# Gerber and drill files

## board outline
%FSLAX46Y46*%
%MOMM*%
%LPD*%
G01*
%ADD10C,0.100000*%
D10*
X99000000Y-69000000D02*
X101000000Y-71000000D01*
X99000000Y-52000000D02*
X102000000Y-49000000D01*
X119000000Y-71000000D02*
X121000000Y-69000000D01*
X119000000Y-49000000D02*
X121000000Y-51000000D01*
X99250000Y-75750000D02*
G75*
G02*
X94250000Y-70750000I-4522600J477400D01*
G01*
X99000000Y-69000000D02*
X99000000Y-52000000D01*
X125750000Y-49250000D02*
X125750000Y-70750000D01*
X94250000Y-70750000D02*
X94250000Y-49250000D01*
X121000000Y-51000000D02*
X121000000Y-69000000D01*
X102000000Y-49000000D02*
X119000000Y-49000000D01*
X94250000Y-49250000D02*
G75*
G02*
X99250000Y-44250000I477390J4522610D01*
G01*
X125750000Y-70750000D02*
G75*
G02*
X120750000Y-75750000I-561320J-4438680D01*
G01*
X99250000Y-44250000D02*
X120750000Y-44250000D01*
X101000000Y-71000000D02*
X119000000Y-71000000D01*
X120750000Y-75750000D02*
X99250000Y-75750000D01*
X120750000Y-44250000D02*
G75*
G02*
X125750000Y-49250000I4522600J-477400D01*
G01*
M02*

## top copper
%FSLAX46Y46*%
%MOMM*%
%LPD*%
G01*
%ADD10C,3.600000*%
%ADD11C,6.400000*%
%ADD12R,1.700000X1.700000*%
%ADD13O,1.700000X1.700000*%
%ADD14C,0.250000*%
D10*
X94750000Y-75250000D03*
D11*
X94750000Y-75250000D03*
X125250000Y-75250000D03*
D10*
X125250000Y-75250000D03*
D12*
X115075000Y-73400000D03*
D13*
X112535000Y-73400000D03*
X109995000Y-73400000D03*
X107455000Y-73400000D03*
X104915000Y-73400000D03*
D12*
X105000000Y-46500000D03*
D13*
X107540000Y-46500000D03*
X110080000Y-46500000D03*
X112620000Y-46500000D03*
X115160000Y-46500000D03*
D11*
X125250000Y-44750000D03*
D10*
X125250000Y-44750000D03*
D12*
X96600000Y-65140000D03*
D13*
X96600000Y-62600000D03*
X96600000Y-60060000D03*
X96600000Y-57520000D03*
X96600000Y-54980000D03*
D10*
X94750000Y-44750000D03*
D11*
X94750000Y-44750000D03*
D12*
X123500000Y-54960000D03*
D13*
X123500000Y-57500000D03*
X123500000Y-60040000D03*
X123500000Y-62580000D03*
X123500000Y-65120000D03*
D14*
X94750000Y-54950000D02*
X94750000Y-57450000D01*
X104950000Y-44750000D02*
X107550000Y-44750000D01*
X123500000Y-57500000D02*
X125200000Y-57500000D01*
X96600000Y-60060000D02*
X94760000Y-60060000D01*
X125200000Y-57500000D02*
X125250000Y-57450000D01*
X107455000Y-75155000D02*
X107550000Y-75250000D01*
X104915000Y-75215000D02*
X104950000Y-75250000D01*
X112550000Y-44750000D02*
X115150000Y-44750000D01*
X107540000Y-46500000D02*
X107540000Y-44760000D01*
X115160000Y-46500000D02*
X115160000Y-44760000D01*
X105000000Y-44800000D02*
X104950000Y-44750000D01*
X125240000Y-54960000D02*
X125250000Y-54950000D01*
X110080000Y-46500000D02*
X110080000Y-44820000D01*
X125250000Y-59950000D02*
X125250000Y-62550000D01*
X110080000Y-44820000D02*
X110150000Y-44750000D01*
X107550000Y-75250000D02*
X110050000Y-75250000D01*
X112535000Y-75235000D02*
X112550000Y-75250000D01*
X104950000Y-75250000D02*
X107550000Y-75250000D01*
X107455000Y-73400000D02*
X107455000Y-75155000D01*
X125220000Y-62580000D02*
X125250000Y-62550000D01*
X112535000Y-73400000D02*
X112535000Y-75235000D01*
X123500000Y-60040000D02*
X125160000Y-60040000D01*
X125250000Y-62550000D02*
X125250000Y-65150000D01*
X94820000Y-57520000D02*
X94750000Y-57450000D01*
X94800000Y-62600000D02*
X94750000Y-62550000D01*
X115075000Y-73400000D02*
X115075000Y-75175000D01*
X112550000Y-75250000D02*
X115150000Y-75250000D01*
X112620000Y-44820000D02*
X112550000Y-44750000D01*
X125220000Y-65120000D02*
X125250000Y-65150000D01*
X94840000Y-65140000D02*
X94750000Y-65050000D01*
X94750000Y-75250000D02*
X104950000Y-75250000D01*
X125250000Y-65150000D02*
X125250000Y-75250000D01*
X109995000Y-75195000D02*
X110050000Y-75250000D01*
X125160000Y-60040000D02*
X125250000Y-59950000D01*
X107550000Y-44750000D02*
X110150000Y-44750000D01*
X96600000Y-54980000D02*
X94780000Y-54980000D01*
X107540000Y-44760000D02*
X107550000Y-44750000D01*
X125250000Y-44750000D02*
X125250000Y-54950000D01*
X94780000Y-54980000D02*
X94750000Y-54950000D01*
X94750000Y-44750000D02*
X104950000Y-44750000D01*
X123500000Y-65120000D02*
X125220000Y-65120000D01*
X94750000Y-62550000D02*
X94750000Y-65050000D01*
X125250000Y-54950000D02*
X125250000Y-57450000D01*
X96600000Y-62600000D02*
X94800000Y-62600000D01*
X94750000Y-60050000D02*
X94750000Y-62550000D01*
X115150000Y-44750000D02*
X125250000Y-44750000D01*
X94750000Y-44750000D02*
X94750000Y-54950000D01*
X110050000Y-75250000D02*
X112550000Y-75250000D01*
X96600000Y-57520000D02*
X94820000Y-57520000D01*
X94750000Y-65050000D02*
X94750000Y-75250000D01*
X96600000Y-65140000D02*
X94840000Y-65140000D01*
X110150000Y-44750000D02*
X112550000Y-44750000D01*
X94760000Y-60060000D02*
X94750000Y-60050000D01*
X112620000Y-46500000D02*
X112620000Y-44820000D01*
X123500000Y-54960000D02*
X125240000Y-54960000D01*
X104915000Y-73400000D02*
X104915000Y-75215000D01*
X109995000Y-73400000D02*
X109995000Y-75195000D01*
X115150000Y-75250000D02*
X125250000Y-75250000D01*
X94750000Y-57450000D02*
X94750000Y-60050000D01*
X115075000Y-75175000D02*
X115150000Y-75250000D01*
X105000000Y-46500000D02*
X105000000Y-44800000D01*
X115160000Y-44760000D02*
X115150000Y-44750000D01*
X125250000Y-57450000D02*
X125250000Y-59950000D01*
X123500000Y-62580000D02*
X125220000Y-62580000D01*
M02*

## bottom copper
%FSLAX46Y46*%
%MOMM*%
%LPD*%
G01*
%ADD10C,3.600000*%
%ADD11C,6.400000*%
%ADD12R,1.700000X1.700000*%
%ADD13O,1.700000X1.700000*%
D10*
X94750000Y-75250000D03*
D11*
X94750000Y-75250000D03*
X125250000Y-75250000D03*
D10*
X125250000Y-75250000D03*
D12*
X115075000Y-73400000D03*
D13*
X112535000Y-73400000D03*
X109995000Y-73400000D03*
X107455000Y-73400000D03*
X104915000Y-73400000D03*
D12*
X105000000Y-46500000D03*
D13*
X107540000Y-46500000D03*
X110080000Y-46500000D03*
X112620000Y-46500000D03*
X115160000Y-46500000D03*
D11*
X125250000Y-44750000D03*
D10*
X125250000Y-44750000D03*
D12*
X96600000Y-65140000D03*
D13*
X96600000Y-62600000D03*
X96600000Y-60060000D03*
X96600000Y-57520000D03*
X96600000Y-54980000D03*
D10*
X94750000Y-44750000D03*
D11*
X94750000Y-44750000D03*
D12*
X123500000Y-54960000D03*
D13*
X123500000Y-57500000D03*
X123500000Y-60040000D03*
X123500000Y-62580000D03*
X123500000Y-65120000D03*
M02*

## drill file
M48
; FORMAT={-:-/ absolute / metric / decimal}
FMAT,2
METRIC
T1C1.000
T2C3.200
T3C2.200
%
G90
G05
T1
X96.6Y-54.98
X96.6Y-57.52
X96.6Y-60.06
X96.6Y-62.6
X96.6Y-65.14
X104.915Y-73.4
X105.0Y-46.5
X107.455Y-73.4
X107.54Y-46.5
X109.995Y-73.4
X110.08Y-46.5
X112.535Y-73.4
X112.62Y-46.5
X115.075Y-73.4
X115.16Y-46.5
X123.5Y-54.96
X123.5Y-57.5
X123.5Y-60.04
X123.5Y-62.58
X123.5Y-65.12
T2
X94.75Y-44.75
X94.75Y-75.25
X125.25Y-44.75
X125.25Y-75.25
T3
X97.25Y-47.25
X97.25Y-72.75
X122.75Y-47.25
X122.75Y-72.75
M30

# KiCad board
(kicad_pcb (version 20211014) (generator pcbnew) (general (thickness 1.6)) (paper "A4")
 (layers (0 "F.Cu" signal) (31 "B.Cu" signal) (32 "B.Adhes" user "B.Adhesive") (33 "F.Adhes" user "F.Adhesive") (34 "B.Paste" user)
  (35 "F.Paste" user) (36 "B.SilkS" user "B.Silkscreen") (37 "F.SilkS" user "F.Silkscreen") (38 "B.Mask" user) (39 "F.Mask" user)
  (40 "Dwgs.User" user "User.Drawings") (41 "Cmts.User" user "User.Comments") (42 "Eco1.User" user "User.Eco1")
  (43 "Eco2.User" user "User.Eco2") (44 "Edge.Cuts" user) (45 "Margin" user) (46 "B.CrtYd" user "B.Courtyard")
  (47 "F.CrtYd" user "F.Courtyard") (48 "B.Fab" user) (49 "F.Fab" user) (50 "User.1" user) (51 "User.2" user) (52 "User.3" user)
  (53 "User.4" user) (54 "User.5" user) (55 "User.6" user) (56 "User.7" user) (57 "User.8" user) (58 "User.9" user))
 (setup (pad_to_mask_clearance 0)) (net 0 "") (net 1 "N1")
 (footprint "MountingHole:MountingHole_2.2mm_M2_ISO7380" (layer "F.Cu") (at 122.75 47.25)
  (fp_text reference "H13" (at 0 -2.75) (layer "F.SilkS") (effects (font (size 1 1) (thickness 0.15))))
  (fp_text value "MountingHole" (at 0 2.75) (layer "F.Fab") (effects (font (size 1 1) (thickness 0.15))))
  (pad "" np_thru_hole circle (at 0 0) (size 2.2 2.2) (drill 2.2) (layers *.Cu *.Mask)))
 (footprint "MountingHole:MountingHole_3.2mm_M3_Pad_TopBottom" (layer "F.Cu") (at 94.75 75.25)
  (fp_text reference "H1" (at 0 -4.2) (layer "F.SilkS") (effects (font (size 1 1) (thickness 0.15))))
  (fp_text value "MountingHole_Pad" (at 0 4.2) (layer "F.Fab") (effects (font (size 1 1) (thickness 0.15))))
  (pad "1" thru_hole circle (at 0 0) (size 3.6 3.6) (drill 3.2) (layers *.Cu *.Mask) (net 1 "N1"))
  (pad "1" connect circle (at 0 0) (size 6.4 6.4) (layers "B.Cu" "B.Mask") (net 1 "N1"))
  (pad "1" connect circle (at 0 0) (size 6.4 6.4) (layers "F.Cu" "F.Mask") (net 1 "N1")))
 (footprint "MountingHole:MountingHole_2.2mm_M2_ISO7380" (layer "F.Cu") (at 97.25 72.75)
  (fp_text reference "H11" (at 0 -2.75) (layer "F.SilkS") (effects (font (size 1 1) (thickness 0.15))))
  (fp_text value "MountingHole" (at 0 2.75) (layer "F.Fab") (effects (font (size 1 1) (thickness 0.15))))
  (pad "" np_thru_hole circle (at 0 0) (size 2.2 2.2) (drill 2.2) (layers *.Cu *.Mask)))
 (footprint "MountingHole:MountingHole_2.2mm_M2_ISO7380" (layer "F.Cu") (at 97.25 47.25)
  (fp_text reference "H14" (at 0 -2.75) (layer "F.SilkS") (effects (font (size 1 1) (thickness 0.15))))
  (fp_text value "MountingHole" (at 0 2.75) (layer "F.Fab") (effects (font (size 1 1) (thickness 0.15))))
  (pad "" np_thru_hole circle (at 0 0) (size 2.2 2.2) (drill 2.2) (layers *.Cu *.Mask)))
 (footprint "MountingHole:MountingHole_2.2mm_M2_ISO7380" (layer "F.Cu") (at 122.75 72.75)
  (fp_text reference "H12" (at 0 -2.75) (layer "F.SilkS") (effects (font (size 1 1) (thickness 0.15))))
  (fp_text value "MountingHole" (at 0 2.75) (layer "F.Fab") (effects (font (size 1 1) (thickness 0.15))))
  (pad "" np_thru_hole circle (at 0 0) (size 2.2 2.2) (drill 2.2) (layers *.Cu *.Mask)))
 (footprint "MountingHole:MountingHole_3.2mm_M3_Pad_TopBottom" (layer "F.Cu") (at 125.25 75.25)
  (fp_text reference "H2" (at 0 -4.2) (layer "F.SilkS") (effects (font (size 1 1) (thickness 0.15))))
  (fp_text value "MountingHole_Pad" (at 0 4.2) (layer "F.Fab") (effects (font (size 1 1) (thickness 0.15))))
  (pad "1" connect circle (at 0 0) (size 6.4 6.4) (layers "B.Cu" "B.Mask") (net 1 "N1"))
  (pad "1" connect circle (at 0 0) (size 6.4 6.4) (layers "F.Cu" "F.Mask") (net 1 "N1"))
  (pad "1" thru_hole circle (at 0 0) (size 3.6 3.6) (drill 3.2) (layers *.Cu *.Mask) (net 1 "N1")))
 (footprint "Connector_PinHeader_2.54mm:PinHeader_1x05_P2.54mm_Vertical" (layer "F.Cu") (at 115.075 73.4 -90)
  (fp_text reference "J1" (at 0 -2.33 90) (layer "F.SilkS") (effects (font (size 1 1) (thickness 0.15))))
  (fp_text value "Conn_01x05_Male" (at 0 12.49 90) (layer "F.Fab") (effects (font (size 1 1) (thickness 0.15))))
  (pad "1" thru_hole rect (at 0 0 270) (size 1.7 1.7) (drill 1) (layers *.Cu *.Mask) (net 1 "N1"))
  (pad "2" thru_hole oval (at 0 2.54 270) (size 1.7 1.7) (drill 1) (layers *.Cu *.Mask) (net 1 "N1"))
  (pad "3" thru_hole oval (at 0 5.08 270) (size 1.7 1.7) (drill 1) (layers *.Cu *.Mask) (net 1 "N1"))
  (pad "4" thru_hole oval (at 0 7.62 270) (size 1.7 1.7) (drill 1) (layers *.Cu *.Mask) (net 1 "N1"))
  (pad "5" thru_hole oval (at 0 10.16 270) (size 1.7 1.7) (drill 1) (layers *.Cu *.Mask) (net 1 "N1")))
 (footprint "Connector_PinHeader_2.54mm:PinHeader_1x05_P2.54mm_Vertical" (layer "F.Cu") (at 105 46.5 90)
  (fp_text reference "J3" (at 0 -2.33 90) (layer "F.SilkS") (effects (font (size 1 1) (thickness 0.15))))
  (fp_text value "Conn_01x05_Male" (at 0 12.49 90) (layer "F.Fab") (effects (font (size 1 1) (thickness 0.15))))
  (pad "1" thru_hole rect (at 0 0 90) (size 1.7 1.7) (drill 1) (layers *.Cu *.Mask) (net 1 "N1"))
  (pad "2" thru_hole oval (at 0 2.54 90) (size 1.7 1.7) (drill 1) (layers *.Cu *.Mask) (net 1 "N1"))
  (pad "3" thru_hole oval (at 0 5.08 90) (size 1.7 1.7) (drill 1) (layers *.Cu *.Mask) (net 1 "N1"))
  (pad "4" thru_hole oval (at 0 7.62 90) (size 1.7 1.7) (drill 1) (layers *.Cu *.Mask) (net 1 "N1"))
  (pad "5" thru_hole oval (at 0 10.16 90) (size 1.7 1.7) (drill 1) (layers *.Cu *.Mask) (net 1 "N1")))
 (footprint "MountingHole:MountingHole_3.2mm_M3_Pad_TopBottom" (layer "F.Cu") (at 125.25 44.75)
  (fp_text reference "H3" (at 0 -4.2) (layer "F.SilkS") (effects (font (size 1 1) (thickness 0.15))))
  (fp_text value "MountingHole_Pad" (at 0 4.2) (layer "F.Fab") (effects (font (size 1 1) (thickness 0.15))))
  (pad "1" connect circle (at 0 0) (size 6.4 6.4) (layers "F.Cu" "F.Mask") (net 1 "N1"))
  (pad "1" connect circle (at 0 0) (size 6.4 6.4) (layers "B.Cu" "B.Mask") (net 1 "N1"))
  (pad "1" thru_hole circle (at 0 0) (size 3.6 3.6) (drill 3.2) (layers *.Cu *.Mask) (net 1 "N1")))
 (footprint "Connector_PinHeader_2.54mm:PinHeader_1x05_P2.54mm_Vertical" (layer "F.Cu") (at 96.6 65.14 180)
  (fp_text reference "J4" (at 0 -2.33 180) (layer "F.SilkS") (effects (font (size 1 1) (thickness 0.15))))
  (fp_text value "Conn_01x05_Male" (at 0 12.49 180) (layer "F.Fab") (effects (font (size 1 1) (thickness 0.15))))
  (pad "1" thru_hole rect (at 0 0 180) (size 1.7 1.7) (drill 1) (layers *.Cu *.Mask) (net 1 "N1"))
  (pad "2" thru_hole oval (at 0 2.54 180) (size 1.7 1.7) (drill 1) (layers *.Cu *.Mask) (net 1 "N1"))
  (pad "3" thru_hole oval (at 0 5.08 180) (size 1.7 1.7) (drill 1) (layers *.Cu *.Mask) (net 1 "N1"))
  (pad "4" thru_hole oval (at 0 7.62 180) (size 1.7 1.7) (drill 1) (layers *.Cu *.Mask) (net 1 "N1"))
  (pad "5" thru_hole oval (at 0 10.16 180) (size 1.7 1.7) (drill 1) (layers *.Cu *.Mask) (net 1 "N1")))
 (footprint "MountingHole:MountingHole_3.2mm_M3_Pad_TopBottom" (layer "F.Cu") (at 94.75 44.75)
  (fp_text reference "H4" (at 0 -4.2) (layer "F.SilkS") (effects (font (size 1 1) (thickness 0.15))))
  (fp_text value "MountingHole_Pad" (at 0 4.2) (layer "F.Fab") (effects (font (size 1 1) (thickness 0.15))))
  (pad "1" thru_hole circle (at 0 0) (size 3.6 3.6) (drill 3.2) (layers *.Cu *.Mask) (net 1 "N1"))
  (pad "1" connect circle (at 0 0) (size 6.4 6.4) (layers "F.Cu" "F.Mask") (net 1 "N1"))
  (pad "1" connect circle (at 0 0) (size 6.4 6.4) (layers "B.Cu" "B.Mask") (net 1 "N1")))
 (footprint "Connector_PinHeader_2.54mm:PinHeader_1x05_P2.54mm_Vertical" (layer "F.Cu") (at 123.5 54.96)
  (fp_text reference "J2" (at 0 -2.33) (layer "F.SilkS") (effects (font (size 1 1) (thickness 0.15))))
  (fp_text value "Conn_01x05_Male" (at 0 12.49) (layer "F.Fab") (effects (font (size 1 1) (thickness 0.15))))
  (pad "1" thru_hole rect (at 0 0) (size 1.7 1.7) (drill 1) (layers *.Cu *.Mask) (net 1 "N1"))
  (pad "2" thru_hole oval (at 0 2.54) (size 1.7 1.7) (drill 1) (layers *.Cu *.Mask) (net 1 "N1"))
  (pad "3" thru_hole oval (at 0 5.08) (size 1.7 1.7) (drill 1) (layers *.Cu *.Mask) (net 1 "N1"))
  (pad "4" thru_hole oval (at 0 7.62) (size 1.7 1.7) (drill 1) (layers *.Cu *.Mask) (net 1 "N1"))
  (pad "5" thru_hole oval (at 0 10.16) (size 1.7 1.7) (drill 1) (layers *.Cu *.Mask) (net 1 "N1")))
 (gr_line (start 99 69) (end 101 71) (layer "Edge.Cuts") (width 0.1))
 (gr_line (start 99 52) (end 102 49) (layer "Edge.Cuts") (width 0.1))
 (gr_line (start 119 71) (end 121 69) (layer "Edge.Cuts") (width 0.1))
 (gr_line (start 119 49) (end 121 51) (layer "Edge.Cuts") (width 0.1))
 (gr_arc (start 99.25 75.75) (mid 91.511648 78.48835) (end 94.25 70.75) (layer "Edge.Cuts") (width 0.1))
 (gr_line (start 99 69) (end 99 52) (layer "Edge.Cuts") (width 0.1))
 (gr_line (start 125.75 49.25) (end 125.75 70.75) (layer "Edge.Cuts") (width 0.1))
 (gr_line (start 94.25 70.75) (end 94.25 49.25) (layer "Edge.Cuts") (width 0.1))
 (gr_line (start 121 51) (end 121 69) (layer "Edge.Cuts") (width 0.1))
 (gr_line (start 102 49) (end 119 49) (layer "Edge.Cuts") (width 0.1))
 (gr_arc (start 94.25 49.25) (mid 91.511649 41.511649) (end 99.25 44.25) (layer "Edge.Cuts") (width 0.1))
 (gr_arc (start 125.75 70.75) (mid 128.352298 78.352298) (end 120.75 75.75) (layer "Edge.Cuts") (width 0.1))
 (gr_line (start 99.25 44.25) (end 120.75 44.25) (layer "Edge.Cuts") (width 0.1))
 (gr_line (start 101 71) (end 119 71) (layer "Edge.Cuts") (width 0.1))
 (gr_line (start 120.75 75.75) (end 99.25 75.75) (layer "Edge.Cuts") (width 0.1))
 (gr_arc (start 120.75 44.25) (mid 128.488349 41.511649) (end 125.75 49.25) (layer "Edge.Cuts") (width 0.1))
 (segment (start 94.75 54.95) (end 94.75 57.45) (width 0.25) (layer "F.Cu") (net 1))
 (segment (start 104.95 44.75) (end 107.55 44.75) (width 0.25) (layer "F.Cu") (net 1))
 (segment (start 123.5 57.5) (end 125.2 57.5) (width 0.25) (layer "F.Cu") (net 1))
 (segment (start 96.6 60.06) (end 94.76 60.06) (width 0.25) (layer "F.Cu") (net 1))
 (segment (start 125.2 57.5) (end 125.25 57.45) (width 0.25) (layer "F.Cu") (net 1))
 (segment (start 107.455 75.155) (end 107.55 75.25) (width 0.25) (layer "F.Cu") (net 1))
 (segment (start 104.915 75.215) (end 104.95 75.25) (width 0.25) (layer "F.Cu") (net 1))
 (segment (start 112.55 44.75) (end 115.15 44.75) (width 0.25) (layer "F.Cu") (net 1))
 (segment (start 107.54 46.5) (end 107.54 44.76) (width 0.25) (layer "F.Cu") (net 1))
 (segment (start 115.16 46.5) (end 115.16 44.76) (width 0.25) (layer "F.Cu") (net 1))
 (segment (start 105 44.8) (end 104.95 44.75) (width 0.25) (layer "F.Cu") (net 1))
 (segment (start 125.24 54.96) (end 125.25 54.95) (width 0.25) (layer "F.Cu") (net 1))
 (segment (start 110.08 46.5) (end 110.08 44.82) (width 0.25) (layer "F.Cu") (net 1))
 (segment (start 125.25 59.95) (end 125.25 62.55) (width 0.25) (layer "F.Cu") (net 1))
 (segment (start 110.08 44.82) (end 110.15 44.75) (width 0.25) (layer "F.Cu") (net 1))
 (segment (start 107.55 75.25) (end 110.05 75.25) (width 0.25) (layer "F.Cu") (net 1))
 (segment (start 112.535 75.235) (end 112.55 75.25) (width 0.25) (layer "F.Cu") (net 1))
 (segment (start 104.95 75.25) (end 107.55 75.25) (width 0.25) (layer "F.Cu") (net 1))
 (segment (start 107.455 73.4) (end 107.455 75.155) (width 0.25) (layer "F.Cu") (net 1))
 (segment (start 125.22 62.58) (end 125.25 62.55) (width 0.25) (layer "F.Cu") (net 1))
 (segment (start 112.535 73.4) (end 112.535 75.235) (width 0.25) (layer "F.Cu") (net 1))
 (segment (start 123.5 60.04) (end 125.16 60.04) (width 0.25) (layer "F.Cu") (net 1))
 (segment (start 125.25 62.55) (end 125.25 65.15) (width 0.25) (layer "F.Cu") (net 1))
 (segment (start 94.82 57.52) (end 94.75 57.45) (width 0.25) (layer "F.Cu") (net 1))
 (segment (start 94.8 62.6) (end 94.75 62.55) (width 0.25) (layer "F.Cu") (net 1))
 (segment (start 115.075 73.4) (end 115.075 75.175) (width 0.25) (layer "F.Cu") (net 1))
 (segment (start 112.55 75.25) (end 115.15 75.25) (width 0.25) (layer "F.Cu") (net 1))
 (segment (start 112.62 44.82) (end 112.55 44.75) (width 0.25) (layer "F.Cu") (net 1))
 (segment (start 125.22 65.12) (end 125.25 65.15) (width 0.25) (layer "F.Cu") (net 1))
 (segment (start 94.84 65.14) (end 94.75 65.05) (width 0.25) (layer "F.Cu") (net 1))
 (segment (start 94.75 75.25) (end 104.95 75.25) (width 0.25) (layer "F.Cu") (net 1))
 (segment (start 125.25 65.15) (end 125.25 75.25) (width 0.25) (layer "F.Cu") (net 1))
 (segment (start 109.995 75.195) (end 110.05 75.25) (width 0.25) (layer "F.Cu") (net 1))
 (segment (start 125.16 60.04) (end 125.25 59.95) (width 0.25) (layer "F.Cu") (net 1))
 (segment (start 107.55 44.75) (end 110.15 44.75) (width 0.25) (layer "F.Cu") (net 1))
 (segment (start 96.6 54.98) (end 94.78 54.98) (width 0.25) (layer "F.Cu") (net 1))
 (segment (start 107.54 44.76) (end 107.55 44.75) (width 0.25) (layer "F.Cu") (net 1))
 (segment (start 125.25 44.75) (end 125.25 54.95) (width 0.25) (layer "F.Cu") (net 1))
 (segment (start 94.78 54.98) (end 94.75 54.95) (width 0.25) (layer "F.Cu") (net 1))
 (segment (start 94.75 44.75) (end 104.95 44.75) (width 0.25) (layer "F.Cu") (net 1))
 (segment (start 123.5 65.12) (end 125.22 65.12) (width 0.25) (layer "F.Cu") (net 1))
 (segment (start 94.75 62.55) (end 94.75 65.05) (width 0.25) (layer "F.Cu") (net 1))
 (segment (start 125.25 54.95) (end 125.25 57.45) (width 0.25) (layer "F.Cu") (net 1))
 (segment (start 96.6 62.6) (end 94.8 62.6) (width 0.25) (layer "F.Cu") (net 1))
 (segment (start 94.75 60.05) (end 94.75 62.55) (width 0.25) (layer "F.Cu") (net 1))
 (segment (start 115.15 44.75) (end 125.25 44.75) (width 0.25) (layer "F.Cu") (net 1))
 (segment (start 94.75 44.75) (end 94.75 54.95) (width 0.25) (layer "F.Cu") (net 1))
 (segment (start 110.05 75.25) (end 112.55 75.25) (width 0.25) (layer "F.Cu") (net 1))
 (segment (start 96.6 57.52) (end 94.82 57.52) (width 0.25) (layer "F.Cu") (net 1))
 (segment (start 94.75 65.05) (end 94.75 75.25) (width 0.25) (layer "F.Cu") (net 1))
 (segment (start 96.6 65.14) (end 94.84 65.14) (width 0.25) (layer "F.Cu") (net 1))
 (segment (start 110.15 44.75) (end 112.55 44.75) (width 0.25) (layer "F.Cu") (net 1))
 (segment (start 94.76 60.06) (end 94.75 60.05) (width 0.25) (layer "F.Cu") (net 1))
 (segment (start 112.62 46.5) (end 112.62 44.82) (width 0.25) (layer "F.Cu") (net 1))
 (segment (start 123.5 54.96) (end 125.24 54.96) (width 0.25) (layer "F.Cu") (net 1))
 (segment (start 104.915 73.4) (end 104.915 75.215) (width 0.25) (layer "F.Cu") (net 1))
 (segment (start 109.995 73.4) (end 109.995 75.195) (width 0.25) (layer "F.Cu") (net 1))
 (segment (start 115.15 75.25) (end 125.25 75.25) (width 0.25) (layer "F.Cu") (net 1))
 (segment (start 94.75 57.45) (end 94.75 60.05) (width 0.25) (layer "F.Cu") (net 1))
 (segment (start 115.075 75.175) (end 115.15 75.25) (width 0.25) (layer "F.Cu") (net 1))
 (segment (start 105 46.5) (end 105 44.8) (width 0.25) (layer "F.Cu") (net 1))
 (segment (start 115.16 44.76) (end 115.15 44.75) (width 0.25) (layer "F.Cu") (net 1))
 (segment (start 125.25 57.45) (end 125.25 59.95) (width 0.25) (layer "F.Cu") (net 1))
 (segment (start 123.5 62.58) (end 125.22 62.58) (width 0.25) (layer "F.Cu") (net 1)))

